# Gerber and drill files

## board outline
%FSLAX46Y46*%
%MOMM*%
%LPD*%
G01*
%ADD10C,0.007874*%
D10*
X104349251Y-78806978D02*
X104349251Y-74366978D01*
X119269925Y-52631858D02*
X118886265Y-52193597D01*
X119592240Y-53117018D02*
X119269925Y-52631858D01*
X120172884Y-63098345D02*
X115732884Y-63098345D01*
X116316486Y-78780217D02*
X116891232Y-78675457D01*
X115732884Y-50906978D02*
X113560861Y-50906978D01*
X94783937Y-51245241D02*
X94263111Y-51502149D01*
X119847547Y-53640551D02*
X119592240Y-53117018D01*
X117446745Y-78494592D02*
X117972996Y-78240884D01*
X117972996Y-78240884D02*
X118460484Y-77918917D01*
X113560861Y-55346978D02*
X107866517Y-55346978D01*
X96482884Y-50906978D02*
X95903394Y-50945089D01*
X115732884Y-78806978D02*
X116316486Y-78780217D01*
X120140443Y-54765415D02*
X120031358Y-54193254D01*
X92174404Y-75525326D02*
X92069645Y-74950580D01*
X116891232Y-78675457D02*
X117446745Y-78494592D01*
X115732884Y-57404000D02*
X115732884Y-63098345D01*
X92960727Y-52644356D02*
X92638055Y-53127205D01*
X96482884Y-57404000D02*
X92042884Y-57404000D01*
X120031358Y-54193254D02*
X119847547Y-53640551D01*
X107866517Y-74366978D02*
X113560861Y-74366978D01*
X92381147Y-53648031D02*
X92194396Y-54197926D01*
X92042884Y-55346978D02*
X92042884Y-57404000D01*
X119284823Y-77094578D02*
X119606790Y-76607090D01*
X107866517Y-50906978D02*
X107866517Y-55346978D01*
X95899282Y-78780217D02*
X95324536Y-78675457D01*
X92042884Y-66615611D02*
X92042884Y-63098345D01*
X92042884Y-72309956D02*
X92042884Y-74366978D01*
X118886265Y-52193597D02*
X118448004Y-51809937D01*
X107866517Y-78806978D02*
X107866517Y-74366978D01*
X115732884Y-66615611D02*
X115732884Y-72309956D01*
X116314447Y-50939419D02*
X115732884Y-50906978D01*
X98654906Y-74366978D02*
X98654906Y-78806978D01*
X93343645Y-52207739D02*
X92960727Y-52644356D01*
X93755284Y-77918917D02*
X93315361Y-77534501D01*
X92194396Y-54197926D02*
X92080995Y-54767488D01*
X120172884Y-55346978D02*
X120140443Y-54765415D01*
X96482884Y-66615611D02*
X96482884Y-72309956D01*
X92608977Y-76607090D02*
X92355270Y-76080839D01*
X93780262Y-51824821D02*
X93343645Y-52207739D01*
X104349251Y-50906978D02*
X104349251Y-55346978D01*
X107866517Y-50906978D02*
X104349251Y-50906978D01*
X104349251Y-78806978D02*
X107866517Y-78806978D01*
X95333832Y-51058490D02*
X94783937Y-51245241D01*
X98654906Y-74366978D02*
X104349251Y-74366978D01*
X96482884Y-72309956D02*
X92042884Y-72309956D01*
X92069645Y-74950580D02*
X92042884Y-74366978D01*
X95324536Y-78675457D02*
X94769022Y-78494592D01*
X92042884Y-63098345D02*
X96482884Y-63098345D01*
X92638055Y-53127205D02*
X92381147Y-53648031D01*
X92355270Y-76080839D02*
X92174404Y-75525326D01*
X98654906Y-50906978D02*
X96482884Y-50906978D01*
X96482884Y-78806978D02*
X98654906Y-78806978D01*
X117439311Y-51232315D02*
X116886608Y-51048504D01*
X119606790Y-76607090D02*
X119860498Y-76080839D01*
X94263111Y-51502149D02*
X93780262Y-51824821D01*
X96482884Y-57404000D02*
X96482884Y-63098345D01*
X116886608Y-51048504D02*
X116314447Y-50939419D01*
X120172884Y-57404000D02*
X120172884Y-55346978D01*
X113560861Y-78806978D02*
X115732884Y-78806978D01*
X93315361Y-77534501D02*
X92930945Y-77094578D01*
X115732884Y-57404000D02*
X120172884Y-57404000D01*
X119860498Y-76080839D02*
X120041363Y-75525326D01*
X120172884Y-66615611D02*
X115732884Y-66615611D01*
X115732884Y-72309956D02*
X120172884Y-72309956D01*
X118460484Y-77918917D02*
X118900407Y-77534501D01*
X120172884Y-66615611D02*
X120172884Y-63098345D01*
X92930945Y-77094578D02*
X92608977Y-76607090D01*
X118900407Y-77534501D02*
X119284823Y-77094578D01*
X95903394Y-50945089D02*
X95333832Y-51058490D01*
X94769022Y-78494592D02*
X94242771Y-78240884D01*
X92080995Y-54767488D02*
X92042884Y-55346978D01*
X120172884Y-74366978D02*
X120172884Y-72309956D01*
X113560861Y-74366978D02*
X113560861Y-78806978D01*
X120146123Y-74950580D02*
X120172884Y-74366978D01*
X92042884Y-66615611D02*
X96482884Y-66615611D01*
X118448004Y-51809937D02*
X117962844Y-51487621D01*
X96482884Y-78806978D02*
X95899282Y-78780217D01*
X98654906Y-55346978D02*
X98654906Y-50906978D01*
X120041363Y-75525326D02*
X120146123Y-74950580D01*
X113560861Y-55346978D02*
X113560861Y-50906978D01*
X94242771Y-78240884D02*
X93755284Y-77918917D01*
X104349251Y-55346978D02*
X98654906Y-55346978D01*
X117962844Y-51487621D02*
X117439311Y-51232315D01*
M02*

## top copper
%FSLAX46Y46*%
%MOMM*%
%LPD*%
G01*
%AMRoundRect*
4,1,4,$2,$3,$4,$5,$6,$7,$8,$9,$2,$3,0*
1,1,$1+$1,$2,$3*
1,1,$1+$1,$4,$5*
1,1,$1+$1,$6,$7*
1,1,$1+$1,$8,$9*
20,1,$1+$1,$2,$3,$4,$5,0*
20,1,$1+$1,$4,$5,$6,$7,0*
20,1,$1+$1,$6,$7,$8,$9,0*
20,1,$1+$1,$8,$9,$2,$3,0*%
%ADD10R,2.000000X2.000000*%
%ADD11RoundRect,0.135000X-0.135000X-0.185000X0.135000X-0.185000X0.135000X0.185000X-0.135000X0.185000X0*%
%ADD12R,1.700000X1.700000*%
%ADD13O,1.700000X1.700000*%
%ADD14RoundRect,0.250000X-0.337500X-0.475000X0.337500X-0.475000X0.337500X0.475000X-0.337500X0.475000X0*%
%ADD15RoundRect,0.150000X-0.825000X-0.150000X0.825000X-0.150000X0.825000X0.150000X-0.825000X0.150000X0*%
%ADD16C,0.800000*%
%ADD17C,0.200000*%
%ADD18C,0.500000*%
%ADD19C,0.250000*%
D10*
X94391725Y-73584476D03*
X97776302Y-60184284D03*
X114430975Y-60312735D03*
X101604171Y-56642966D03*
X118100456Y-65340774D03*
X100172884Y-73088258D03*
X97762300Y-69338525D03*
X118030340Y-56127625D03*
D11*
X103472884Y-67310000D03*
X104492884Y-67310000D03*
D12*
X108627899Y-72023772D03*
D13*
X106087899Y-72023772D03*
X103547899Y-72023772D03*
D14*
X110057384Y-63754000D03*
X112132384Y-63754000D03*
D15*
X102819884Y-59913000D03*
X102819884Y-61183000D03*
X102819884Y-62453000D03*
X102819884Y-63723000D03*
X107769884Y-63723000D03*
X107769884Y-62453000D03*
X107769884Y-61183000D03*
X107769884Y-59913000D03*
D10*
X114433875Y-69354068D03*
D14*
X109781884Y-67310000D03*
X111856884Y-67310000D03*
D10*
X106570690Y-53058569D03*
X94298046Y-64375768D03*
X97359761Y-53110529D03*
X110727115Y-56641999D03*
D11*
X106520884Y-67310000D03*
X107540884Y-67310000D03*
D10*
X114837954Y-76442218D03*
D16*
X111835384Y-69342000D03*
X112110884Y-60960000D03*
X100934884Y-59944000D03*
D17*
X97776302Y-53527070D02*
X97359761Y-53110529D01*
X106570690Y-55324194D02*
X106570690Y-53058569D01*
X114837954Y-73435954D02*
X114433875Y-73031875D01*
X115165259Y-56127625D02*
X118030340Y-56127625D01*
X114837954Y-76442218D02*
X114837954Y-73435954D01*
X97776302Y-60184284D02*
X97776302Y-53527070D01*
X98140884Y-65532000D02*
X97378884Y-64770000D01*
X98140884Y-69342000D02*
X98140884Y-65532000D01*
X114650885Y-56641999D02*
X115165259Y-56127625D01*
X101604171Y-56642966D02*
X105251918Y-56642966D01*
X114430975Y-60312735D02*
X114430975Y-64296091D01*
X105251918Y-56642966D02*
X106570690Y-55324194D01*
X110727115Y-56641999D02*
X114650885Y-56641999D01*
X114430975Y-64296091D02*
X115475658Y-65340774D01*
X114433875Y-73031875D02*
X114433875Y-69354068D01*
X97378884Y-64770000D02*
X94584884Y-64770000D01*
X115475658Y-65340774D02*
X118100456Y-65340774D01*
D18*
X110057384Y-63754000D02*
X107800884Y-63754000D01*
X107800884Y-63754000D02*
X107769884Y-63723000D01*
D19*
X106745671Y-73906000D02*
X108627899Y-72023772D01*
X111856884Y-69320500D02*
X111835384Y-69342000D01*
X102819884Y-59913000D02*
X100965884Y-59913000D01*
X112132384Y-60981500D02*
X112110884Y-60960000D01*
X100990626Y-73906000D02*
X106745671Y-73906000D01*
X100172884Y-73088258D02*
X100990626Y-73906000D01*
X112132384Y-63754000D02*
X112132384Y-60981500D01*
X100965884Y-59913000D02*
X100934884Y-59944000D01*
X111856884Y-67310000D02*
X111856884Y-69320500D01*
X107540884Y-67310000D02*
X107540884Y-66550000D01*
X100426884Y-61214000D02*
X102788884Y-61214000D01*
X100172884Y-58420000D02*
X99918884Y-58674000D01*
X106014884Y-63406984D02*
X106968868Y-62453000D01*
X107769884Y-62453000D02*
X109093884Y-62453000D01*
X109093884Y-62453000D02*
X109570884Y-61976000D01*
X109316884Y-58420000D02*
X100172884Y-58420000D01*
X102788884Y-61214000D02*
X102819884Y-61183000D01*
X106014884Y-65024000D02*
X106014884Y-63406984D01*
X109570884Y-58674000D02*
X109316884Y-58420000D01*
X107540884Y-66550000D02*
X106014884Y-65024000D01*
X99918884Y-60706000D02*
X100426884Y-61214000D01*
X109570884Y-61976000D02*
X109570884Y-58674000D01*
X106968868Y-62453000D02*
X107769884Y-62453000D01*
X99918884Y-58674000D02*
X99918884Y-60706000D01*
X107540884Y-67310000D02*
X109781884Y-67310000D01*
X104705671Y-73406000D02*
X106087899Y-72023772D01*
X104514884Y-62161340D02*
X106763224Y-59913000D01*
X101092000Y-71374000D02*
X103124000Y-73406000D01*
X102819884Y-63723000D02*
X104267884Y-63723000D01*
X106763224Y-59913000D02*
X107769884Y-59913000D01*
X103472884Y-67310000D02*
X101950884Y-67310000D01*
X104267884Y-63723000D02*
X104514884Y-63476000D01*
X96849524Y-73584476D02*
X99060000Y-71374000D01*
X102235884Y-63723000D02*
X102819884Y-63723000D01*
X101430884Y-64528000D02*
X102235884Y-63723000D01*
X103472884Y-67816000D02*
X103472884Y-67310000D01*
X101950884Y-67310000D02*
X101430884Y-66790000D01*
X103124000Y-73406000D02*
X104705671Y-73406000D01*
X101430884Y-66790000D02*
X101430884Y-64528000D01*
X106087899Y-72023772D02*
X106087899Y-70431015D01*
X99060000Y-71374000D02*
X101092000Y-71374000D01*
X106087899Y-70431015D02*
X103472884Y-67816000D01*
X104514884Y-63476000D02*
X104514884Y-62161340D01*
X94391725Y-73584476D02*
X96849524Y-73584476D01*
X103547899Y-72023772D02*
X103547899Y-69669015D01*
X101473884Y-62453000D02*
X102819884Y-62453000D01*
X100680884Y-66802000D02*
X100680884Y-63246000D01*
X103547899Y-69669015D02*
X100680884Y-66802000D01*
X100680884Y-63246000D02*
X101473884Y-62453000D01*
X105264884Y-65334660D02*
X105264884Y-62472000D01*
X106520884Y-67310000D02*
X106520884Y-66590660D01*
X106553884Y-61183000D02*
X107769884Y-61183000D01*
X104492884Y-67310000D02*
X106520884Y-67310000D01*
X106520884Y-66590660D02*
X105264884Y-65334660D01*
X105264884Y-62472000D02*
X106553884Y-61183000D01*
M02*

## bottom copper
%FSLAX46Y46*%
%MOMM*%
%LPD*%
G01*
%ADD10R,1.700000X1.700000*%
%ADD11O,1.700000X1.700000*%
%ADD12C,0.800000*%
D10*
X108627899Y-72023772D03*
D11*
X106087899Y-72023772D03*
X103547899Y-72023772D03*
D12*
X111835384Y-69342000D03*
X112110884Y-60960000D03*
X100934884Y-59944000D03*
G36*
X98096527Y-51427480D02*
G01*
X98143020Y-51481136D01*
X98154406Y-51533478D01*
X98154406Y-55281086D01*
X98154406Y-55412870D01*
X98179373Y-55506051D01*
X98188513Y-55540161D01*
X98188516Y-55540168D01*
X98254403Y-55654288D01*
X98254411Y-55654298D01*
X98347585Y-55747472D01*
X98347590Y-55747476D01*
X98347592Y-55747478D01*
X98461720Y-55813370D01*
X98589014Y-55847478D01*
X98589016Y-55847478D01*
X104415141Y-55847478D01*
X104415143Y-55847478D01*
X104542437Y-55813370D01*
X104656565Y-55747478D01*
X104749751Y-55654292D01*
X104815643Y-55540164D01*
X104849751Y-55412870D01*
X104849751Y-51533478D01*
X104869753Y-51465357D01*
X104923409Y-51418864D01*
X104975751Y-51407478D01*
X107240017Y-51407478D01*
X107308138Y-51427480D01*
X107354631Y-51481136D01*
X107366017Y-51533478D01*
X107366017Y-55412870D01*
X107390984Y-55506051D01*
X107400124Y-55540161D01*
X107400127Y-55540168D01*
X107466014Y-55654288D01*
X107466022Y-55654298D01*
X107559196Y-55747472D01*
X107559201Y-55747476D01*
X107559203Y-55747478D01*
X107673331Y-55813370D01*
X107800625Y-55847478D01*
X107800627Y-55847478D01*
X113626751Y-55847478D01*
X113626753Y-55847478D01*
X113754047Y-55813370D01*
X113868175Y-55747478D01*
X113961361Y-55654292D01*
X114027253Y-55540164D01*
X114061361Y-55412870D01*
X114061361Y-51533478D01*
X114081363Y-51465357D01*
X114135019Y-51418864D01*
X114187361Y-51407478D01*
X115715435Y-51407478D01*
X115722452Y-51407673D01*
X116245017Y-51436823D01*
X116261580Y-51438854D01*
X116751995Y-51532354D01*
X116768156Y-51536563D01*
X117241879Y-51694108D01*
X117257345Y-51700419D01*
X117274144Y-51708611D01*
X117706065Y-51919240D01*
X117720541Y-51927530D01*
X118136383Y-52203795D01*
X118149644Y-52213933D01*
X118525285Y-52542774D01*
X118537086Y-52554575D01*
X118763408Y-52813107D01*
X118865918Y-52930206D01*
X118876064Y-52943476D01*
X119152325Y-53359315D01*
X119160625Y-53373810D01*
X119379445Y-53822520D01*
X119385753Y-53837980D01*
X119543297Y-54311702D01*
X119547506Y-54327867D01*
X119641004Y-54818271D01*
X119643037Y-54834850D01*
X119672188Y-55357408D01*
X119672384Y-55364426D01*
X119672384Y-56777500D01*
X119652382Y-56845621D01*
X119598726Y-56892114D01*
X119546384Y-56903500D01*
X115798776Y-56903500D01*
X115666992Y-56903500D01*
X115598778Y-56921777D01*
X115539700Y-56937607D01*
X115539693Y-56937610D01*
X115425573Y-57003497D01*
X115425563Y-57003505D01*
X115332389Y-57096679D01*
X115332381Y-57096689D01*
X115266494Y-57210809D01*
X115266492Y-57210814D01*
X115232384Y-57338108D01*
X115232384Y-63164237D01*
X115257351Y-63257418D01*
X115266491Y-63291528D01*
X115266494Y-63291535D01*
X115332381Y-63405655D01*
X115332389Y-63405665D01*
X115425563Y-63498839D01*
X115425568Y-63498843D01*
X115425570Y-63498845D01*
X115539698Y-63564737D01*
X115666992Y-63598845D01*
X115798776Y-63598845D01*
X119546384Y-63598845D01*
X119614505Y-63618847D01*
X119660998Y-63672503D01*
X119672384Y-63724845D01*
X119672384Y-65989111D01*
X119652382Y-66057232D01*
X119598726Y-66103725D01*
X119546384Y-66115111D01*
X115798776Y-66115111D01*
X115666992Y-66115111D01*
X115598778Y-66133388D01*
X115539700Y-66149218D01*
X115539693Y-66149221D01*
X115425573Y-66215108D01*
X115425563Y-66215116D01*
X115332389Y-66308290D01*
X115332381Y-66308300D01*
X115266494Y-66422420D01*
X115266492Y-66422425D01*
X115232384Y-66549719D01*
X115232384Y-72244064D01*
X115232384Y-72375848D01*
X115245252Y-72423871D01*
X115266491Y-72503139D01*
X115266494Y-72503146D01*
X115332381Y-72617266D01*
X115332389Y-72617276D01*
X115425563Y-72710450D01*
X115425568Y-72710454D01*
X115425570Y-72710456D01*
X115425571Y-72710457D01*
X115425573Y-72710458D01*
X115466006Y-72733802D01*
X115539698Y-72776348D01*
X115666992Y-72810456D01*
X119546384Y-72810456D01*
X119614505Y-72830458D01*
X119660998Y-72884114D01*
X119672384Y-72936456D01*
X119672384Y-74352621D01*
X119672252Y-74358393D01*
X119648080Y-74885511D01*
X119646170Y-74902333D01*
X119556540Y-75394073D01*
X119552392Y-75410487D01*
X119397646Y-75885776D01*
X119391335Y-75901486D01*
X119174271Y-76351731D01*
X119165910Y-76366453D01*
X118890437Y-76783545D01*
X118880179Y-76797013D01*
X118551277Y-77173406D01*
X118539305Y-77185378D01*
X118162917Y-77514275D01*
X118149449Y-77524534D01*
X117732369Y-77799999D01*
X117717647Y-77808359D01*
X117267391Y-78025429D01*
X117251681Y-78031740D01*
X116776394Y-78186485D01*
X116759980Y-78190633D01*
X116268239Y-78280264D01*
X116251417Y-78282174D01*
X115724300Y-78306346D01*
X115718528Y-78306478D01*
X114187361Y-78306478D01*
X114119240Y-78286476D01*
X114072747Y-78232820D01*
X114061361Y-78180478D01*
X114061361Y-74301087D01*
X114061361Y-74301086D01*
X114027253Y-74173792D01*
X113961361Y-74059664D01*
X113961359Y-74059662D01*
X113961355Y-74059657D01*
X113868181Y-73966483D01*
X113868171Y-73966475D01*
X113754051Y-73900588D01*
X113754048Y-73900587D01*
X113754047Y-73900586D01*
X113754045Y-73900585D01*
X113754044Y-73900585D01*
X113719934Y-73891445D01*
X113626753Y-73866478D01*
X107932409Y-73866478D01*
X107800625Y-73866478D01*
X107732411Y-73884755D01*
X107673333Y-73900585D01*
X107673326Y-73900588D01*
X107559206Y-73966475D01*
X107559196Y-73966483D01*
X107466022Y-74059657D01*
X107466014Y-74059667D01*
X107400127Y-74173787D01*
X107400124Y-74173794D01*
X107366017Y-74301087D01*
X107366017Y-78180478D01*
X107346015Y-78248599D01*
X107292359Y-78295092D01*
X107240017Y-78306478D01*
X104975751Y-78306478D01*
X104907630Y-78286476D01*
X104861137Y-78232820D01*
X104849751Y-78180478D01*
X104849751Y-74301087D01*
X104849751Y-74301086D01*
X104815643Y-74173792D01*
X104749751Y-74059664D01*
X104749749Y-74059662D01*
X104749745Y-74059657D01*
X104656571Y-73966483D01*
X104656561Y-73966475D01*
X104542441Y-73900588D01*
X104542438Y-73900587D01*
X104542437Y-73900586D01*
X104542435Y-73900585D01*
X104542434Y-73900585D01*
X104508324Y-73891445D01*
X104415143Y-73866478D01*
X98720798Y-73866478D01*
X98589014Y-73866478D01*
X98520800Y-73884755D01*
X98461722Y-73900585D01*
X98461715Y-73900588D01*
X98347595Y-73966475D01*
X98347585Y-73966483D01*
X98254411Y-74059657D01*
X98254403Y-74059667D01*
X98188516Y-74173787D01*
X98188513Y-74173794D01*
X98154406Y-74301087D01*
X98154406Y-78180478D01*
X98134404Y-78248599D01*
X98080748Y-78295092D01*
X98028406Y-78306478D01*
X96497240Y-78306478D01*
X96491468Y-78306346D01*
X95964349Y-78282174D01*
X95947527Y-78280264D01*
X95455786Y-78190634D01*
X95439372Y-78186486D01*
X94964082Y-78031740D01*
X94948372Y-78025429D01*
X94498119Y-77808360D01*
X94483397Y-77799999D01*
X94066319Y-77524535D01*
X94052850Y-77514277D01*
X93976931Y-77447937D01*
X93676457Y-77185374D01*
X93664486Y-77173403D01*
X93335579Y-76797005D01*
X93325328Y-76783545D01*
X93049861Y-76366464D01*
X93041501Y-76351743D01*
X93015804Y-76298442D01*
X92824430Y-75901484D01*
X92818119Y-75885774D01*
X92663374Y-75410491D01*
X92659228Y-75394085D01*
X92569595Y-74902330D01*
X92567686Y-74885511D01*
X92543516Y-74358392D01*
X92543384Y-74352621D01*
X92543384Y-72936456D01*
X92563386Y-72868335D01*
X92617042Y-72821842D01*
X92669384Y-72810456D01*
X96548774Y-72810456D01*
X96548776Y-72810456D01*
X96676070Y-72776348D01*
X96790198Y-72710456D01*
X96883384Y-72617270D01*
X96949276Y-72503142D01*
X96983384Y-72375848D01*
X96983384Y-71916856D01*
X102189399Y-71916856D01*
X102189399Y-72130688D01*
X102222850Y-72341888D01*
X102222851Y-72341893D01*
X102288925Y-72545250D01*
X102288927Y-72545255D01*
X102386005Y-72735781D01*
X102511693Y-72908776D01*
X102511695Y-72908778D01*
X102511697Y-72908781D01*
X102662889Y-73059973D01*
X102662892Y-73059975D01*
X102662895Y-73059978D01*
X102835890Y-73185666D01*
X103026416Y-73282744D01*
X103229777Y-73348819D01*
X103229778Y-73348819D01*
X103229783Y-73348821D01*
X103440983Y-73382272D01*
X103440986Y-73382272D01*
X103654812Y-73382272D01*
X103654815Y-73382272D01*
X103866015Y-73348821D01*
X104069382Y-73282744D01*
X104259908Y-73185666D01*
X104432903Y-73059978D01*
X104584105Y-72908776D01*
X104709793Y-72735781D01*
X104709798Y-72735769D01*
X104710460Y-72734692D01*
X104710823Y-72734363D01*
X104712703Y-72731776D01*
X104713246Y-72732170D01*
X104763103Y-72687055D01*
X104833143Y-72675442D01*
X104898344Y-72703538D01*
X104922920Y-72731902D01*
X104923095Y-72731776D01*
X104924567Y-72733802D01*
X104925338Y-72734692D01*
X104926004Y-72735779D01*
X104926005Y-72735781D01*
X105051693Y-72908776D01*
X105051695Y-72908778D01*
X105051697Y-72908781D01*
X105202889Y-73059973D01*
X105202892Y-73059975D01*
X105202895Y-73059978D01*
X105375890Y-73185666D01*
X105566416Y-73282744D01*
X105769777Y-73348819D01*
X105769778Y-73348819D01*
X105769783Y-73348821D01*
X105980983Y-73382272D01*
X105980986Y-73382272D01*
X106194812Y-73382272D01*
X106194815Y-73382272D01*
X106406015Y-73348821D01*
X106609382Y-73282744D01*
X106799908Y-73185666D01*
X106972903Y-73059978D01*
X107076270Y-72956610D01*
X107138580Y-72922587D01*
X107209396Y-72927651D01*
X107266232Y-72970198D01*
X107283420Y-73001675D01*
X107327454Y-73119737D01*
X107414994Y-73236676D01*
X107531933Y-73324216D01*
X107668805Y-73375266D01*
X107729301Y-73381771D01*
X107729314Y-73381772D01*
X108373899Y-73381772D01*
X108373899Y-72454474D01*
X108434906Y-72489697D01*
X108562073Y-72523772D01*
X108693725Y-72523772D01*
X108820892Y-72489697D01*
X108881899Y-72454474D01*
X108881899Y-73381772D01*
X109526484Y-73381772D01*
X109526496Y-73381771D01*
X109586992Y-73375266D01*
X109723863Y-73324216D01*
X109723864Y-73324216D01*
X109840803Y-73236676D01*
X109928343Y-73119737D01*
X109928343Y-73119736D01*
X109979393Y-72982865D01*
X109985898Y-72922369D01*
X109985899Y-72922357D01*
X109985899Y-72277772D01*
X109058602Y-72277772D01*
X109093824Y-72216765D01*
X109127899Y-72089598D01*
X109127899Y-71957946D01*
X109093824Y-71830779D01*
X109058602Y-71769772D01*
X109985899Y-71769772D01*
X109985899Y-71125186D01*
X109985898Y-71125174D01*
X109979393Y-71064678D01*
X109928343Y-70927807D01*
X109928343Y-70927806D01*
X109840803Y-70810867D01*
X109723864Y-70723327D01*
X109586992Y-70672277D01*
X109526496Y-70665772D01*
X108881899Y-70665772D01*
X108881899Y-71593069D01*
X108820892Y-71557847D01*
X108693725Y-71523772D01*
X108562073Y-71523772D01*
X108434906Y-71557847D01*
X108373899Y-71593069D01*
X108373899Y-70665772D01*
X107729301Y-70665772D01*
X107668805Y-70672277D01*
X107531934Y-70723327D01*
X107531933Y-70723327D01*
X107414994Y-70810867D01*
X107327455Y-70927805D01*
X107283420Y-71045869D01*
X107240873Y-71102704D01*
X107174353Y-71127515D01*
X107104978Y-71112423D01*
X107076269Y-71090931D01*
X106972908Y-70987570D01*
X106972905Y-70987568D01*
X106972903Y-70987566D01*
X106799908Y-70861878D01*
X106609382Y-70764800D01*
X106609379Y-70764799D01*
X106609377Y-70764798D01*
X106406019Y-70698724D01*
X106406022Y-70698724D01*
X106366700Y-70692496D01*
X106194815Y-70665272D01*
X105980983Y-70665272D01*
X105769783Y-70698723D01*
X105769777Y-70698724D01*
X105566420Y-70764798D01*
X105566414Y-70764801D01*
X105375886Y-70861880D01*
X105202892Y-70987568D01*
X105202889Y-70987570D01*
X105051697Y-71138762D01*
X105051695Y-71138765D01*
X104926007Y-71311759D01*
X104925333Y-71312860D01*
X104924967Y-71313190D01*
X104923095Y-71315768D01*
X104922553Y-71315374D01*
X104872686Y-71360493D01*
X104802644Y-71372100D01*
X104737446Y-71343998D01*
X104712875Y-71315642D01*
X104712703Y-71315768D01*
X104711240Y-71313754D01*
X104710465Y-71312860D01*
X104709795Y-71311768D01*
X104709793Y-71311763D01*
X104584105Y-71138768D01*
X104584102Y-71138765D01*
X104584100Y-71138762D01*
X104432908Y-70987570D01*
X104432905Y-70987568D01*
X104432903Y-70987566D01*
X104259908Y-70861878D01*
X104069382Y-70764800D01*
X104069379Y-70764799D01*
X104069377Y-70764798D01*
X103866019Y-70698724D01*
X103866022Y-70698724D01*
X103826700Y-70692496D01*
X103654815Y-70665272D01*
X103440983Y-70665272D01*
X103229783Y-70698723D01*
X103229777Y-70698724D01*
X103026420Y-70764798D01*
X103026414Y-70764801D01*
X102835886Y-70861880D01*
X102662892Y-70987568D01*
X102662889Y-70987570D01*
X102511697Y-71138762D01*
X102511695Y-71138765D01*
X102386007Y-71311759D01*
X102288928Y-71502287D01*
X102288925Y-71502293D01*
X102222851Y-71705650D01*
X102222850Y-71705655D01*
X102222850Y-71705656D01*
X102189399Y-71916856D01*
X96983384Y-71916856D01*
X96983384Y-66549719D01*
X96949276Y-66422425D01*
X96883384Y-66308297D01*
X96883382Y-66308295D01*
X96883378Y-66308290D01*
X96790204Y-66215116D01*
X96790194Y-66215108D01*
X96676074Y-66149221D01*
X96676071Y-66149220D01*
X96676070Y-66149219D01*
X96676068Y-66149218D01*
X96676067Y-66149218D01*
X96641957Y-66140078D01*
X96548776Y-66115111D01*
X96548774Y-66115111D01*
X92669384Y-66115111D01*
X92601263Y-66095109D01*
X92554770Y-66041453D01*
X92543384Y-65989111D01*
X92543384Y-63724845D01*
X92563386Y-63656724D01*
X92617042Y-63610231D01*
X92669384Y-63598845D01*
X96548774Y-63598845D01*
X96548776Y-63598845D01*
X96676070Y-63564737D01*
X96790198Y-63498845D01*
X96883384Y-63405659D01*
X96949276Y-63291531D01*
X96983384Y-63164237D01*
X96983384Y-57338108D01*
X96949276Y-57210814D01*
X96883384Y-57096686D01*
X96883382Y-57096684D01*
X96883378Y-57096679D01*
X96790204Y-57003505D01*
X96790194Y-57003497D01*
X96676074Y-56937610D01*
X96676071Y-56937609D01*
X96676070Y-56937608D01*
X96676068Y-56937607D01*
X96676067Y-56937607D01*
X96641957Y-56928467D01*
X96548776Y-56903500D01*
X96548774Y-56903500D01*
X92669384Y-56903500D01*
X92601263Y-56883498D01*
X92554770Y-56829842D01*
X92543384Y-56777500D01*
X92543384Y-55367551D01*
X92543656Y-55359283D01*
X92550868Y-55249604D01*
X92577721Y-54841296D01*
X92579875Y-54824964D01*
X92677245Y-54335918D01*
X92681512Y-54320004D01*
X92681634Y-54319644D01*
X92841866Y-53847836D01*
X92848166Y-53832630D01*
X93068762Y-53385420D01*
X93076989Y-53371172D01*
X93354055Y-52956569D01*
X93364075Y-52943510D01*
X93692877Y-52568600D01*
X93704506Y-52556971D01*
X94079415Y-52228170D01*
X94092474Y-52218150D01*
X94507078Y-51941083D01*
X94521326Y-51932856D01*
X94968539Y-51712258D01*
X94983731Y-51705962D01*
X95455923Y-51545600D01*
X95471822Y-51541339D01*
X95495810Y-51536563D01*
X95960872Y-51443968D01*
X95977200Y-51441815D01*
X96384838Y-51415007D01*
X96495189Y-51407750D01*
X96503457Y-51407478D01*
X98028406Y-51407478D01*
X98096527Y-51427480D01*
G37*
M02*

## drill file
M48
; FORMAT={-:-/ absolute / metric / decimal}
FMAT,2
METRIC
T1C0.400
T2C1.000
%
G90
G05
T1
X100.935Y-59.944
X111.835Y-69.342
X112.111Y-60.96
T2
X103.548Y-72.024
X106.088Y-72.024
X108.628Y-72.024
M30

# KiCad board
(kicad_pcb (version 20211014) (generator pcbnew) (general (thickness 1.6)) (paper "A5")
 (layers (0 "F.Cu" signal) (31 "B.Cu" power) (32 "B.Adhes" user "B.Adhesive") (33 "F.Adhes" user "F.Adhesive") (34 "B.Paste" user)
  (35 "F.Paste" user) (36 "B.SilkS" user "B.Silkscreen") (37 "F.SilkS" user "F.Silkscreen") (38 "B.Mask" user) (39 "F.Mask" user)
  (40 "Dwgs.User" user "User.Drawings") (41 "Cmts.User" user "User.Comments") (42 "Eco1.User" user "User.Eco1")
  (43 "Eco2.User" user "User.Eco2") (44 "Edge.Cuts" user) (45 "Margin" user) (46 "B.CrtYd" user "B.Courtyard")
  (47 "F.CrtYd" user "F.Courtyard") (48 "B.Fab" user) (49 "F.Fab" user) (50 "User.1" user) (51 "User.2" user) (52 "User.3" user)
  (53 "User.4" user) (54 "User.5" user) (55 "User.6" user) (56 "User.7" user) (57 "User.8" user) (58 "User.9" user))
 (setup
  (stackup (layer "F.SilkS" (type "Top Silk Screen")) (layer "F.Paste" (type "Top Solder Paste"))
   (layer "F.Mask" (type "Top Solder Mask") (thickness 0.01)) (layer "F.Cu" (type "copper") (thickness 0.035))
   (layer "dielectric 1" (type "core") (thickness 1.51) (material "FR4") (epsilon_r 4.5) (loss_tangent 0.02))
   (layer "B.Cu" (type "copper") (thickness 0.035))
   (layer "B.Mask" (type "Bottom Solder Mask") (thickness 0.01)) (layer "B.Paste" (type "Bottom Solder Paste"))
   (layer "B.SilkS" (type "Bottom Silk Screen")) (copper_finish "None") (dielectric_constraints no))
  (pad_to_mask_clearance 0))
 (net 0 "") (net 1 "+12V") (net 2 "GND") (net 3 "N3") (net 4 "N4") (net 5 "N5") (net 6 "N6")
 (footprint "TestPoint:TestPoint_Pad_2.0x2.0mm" (layer "F.Cu") (at 94.391725 73.584476)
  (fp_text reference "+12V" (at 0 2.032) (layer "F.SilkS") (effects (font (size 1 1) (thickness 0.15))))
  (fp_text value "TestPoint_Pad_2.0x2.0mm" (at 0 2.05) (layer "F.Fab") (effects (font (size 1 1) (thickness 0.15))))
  (pad "1" smd rect (at 0 0) (size 2 2) (layers "F.Cu" "F.Mask") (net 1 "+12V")))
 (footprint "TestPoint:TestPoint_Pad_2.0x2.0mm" (layer "F.Cu") (at 97.776302 60.184284)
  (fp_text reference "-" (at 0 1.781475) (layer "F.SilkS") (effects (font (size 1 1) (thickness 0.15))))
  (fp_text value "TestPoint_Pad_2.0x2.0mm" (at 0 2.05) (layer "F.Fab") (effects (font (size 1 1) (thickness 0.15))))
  (pad "1" smd rect (at 0 0) (size 2 2) (layers "F.Cu" "F.Mask")))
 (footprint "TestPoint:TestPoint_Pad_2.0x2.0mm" (layer "F.Cu") (at 114.430975 60.312735)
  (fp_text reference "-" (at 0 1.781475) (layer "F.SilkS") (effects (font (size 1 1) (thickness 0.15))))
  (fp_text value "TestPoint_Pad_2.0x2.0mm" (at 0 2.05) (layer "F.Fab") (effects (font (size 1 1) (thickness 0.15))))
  (pad "1" smd rect (at 0 0) (size 2 2) (layers "F.Cu" "F.Mask")))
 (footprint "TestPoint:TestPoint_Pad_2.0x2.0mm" (layer "F.Cu") (at 101.604171 56.642966)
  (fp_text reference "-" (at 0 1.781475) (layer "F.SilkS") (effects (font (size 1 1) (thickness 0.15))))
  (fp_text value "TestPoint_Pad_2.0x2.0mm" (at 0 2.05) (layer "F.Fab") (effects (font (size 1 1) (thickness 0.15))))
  (pad "1" smd rect (at 0 0) (size 2 2) (layers "F.Cu" "F.Mask")))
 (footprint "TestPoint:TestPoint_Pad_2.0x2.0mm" (layer "F.Cu") (at 118.100456 65.340774 -90)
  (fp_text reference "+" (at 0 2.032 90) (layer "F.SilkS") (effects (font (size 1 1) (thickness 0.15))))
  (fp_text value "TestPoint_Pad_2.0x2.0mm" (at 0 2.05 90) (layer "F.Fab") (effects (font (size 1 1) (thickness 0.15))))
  (pad "1" smd rect (at 0 0 270) (size 2 2) (layers "F.Cu" "F.Mask")))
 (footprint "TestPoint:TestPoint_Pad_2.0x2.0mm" (layer "F.Cu") (at 100.172884 73.088258 180)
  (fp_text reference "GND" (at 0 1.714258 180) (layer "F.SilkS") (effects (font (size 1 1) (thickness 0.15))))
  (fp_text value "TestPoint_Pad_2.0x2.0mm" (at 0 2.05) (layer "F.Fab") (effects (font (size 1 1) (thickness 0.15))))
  (pad "1" smd rect (at 0 0 180) (size 2 2) (layers "F.Cu" "F.Mask") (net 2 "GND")))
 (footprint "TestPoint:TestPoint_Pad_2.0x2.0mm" (layer "F.Cu") (at 97.7623 69.338525)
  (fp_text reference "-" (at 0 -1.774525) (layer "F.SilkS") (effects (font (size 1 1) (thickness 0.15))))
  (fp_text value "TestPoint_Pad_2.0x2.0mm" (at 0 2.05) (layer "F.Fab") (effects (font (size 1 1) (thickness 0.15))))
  (pad "1" smd rect (at 0 0) (size 2 2) (layers "F.Cu" "F.Mask")))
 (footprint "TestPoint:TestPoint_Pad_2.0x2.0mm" (layer "F.Cu") (at 118.03034 56.127625 -90)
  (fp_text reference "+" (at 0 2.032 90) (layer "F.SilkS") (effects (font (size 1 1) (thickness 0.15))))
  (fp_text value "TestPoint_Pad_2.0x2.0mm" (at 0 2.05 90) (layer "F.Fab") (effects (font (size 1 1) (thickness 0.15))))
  (pad "1" smd rect (at 0 0 270) (size 2 2) (layers "F.Cu" "F.Mask")))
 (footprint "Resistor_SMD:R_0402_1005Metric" (layer "F.Cu") (at 103.982884 67.31)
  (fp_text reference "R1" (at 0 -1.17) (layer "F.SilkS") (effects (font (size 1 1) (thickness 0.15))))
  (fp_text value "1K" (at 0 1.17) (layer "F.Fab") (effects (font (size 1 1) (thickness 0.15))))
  (pad "1" smd roundrect (at -0.51 0) (size 0.54 0.64) (layers "F.Cu" "F.Paste" "F.Mask") (roundrect_rratio 0.25) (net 1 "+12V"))
  (pad "2" smd roundrect (at 0.51 0) (size 0.54 0.64) (layers "F.Cu" "F.Paste" "F.Mask") (roundrect_rratio 0.25) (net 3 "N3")))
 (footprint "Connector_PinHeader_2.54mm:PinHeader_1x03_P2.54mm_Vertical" (layer "F.Cu") (at 108.627899 72.023772 -90)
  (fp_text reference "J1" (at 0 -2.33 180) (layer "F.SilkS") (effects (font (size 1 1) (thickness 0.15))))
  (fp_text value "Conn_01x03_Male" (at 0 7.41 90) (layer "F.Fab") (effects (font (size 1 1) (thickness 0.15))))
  (pad "1" thru_hole rect (at 0 0 270) (size 1.7 1.7) (drill 1) (layers *.Cu *.Mask) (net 2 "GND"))
  (pad "2" thru_hole oval (at 0 2.54 270) (size 1.7 1.7) (drill 1) (layers *.Cu *.Mask) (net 1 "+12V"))
  (pad "3" thru_hole oval (at 0 5.08 270) (size 1.7 1.7) (drill 1) (layers *.Cu *.Mask) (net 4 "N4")))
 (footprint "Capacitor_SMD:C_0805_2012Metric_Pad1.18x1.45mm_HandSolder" (layer "F.Cu") (at 111.094884 63.754)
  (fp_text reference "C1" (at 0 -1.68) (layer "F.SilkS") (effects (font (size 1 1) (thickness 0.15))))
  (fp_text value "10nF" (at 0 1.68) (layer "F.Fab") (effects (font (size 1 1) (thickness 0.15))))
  (pad "1" smd roundrect (at -1.0375 0) (size 1.175 1.45) (layers "F.Cu" "F.Paste" "F.Mask") (roundrect_rratio 0.2127659574) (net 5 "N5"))
  (pad "2" smd roundrect (at 1.0375 0) (size 1.175 1.45) (layers "F.Cu" "F.Paste" "F.Mask") (roundrect_rratio 0.2127659574) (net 2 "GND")))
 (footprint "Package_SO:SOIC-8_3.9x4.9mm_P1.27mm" (layer "F.Cu") (at 105.294884 61.818)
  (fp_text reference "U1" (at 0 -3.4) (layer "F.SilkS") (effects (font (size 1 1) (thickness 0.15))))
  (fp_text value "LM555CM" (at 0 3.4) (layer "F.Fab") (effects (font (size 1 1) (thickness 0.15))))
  (pad "1" smd roundrect (at -2.475 -1.905) (size 1.95 0.6) (layers "F.Cu" "F.Paste" "F.Mask") (roundrect_rratio 0.25) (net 2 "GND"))
  (pad "2" smd roundrect (at -2.475 -0.635) (size 1.95 0.6) (layers "F.Cu" "F.Paste" "F.Mask") (roundrect_rratio 0.25) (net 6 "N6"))
  (pad "3" smd roundrect (at -2.475 0.635) (size 1.95 0.6) (layers "F.Cu" "F.Paste" "F.Mask") (roundrect_rratio 0.25) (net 4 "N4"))
  (pad "4" smd roundrect (at -2.475 1.905) (size 1.95 0.6) (layers "F.Cu" "F.Paste" "F.Mask") (roundrect_rratio 0.25) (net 1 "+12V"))
  (pad "5" smd roundrect (at 2.475 1.905) (size 1.95 0.6) (layers "F.Cu" "F.Paste" "F.Mask") (roundrect_rratio 0.25) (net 5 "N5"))
  (pad "6" smd roundrect (at 2.475 0.635) (size 1.95 0.6) (layers "F.Cu" "F.Paste" "F.Mask") (roundrect_rratio 0.25) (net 6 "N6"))
  (pad "7" smd roundrect (at 2.475 -0.635) (size 1.95 0.6) (layers "F.Cu" "F.Paste" "F.Mask") (roundrect_rratio 0.25) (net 3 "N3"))
  (pad "8" smd roundrect (at 2.475 -1.905) (size 1.95 0.6) (layers "F.Cu" "F.Paste" "F.Mask") (roundrect_rratio 0.25) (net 1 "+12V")))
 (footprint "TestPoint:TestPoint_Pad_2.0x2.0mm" (layer "F.Cu") (at 114.433875 69.354068)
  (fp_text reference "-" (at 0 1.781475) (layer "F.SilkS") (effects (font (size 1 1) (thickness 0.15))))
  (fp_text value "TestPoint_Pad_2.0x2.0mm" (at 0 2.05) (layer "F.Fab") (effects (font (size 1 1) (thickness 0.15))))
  (pad "1" smd rect (at 0 0) (size 2 2) (layers "F.Cu" "F.Mask")))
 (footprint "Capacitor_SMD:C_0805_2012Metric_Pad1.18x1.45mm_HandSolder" (layer "F.Cu") (at 110.819384 67.31)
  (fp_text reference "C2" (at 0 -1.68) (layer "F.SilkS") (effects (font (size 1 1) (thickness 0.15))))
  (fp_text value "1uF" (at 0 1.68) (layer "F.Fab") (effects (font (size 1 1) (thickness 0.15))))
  (pad "1" smd roundrect (at -1.0375 0) (size 1.175 1.45) (layers "F.Cu" "F.Paste" "F.Mask") (roundrect_rratio 0.2127659574) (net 6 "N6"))
  (pad "2" smd roundrect (at 1.0375 0) (size 1.175 1.45) (layers "F.Cu" "F.Paste" "F.Mask") (roundrect_rratio 0.2127659574) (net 2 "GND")))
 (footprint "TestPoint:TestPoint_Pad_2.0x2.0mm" (layer "F.Cu") (at 106.57069 53.058569)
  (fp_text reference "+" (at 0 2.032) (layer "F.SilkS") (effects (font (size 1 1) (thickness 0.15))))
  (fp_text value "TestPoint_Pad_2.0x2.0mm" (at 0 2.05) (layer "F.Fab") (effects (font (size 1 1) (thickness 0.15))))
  (pad "1" smd rect (at 0 0) (size 2 2) (layers "F.Cu" "F.Mask")))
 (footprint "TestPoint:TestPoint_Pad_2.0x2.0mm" (layer "F.Cu") (at 94.298046 64.375768)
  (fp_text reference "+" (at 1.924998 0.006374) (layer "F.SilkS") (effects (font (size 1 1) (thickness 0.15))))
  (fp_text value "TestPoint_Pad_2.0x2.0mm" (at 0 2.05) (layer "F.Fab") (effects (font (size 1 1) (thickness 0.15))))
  (pad "1" smd rect (at 0 0) (size 2 2) (layers "F.Cu" "F.Mask")))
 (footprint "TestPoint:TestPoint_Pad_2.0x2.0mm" (layer "F.Cu") (at 97.359761 53.110529)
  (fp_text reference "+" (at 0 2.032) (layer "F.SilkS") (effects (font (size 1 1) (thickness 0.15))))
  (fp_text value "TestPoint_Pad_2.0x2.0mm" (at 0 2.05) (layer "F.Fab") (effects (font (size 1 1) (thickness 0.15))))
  (pad "1" smd rect (at 0 0) (size 2 2) (layers "F.Cu" "F.Mask")))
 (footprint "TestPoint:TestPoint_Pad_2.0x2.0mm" (layer "F.Cu") (at 110.727115 56.641999)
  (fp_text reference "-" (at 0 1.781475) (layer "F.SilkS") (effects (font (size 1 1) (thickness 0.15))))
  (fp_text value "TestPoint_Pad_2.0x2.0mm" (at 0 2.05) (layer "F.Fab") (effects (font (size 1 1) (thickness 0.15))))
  (pad "1" smd rect (at 0 0) (size 2 2) (layers "F.Cu" "F.Mask")))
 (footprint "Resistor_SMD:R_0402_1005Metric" (layer "F.Cu") (at 107.030884 67.31)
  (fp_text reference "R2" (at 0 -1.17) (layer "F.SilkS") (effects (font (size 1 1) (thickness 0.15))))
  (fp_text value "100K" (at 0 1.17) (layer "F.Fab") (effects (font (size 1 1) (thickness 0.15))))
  (pad "1" smd roundrect (at -0.51 0) (size 0.54 0.64) (layers "F.Cu" "F.Paste" "F.Mask") (roundrect_rratio 0.25) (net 3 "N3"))
  (pad "2" smd roundrect (at 0.51 0) (size 0.54 0.64) (layers "F.Cu" "F.Paste" "F.Mask") (roundrect_rratio 0.25) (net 6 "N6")))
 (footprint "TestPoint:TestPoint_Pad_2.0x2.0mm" (layer "F.Cu") (at 114.837954 76.442218 90)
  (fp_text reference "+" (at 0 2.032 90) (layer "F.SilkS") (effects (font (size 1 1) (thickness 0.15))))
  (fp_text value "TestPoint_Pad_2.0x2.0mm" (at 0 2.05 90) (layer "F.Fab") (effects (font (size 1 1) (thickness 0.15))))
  (pad "1" smd rect (at 0 0 90) (size 2 2) (layers "F.Cu" "F.Mask")))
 (gr_line (start 104.349251 78.806978) (end 104.349251 74.366978) (layer "Edge.Cuts") (width 0.007874))
 (gr_line (start 119.269925 52.631858) (end 118.886265 52.193597) (layer "Edge.Cuts") (width 0.007874))
 (gr_line (start 119.59224 53.117018) (end 119.269925 52.631858) (layer "Edge.Cuts") (width 0.007874))
 (gr_line (start 120.172884 63.098345) (end 115.732884 63.098345) (layer "Edge.Cuts") (width 0.007874))
 (gr_line (start 116.316486 78.780217) (end 116.891232 78.675457) (layer "Edge.Cuts") (width 0.007874))
 (gr_line (start 115.732884 50.906978) (end 113.560861 50.906978) (layer "Edge.Cuts") (width 0.007874))
 (gr_line (start 94.783937 51.245241) (end 94.263111 51.502149) (layer "Edge.Cuts") (width 0.007874))
 (gr_line (start 119.847547 53.640551) (end 119.59224 53.117018) (layer "Edge.Cuts") (width 0.007874))
 (gr_line (start 117.446745 78.494592) (end 117.972996 78.240884) (layer "Edge.Cuts") (width 0.007874))
 (gr_line (start 117.972996 78.240884) (end 118.460484 77.918917) (layer "Edge.Cuts") (width 0.007874))
 (gr_line (start 113.560861 55.346978) (end 107.866517 55.346978) (layer "Edge.Cuts") (width 0.007874))
 (gr_line (start 96.482884 50.906978) (end 95.903394 50.945089) (layer "Edge.Cuts") (width 0.007874))
 (gr_line (start 115.732884 78.806978) (end 116.316486 78.780217) (layer "Edge.Cuts") (width 0.007874))
 (gr_line (start 120.140443 54.765415) (end 120.031358 54.193254) (layer "Edge.Cuts") (width 0.007874))
 (gr_line (start 92.174404 75.525326) (end 92.069645 74.95058) (layer "Edge.Cuts") (width 0.007874))
 (gr_line (start 116.891232 78.675457) (end 117.446745 78.494592) (layer "Edge.Cuts") (width 0.007874))
 (gr_line (start 115.732884 57.404) (end 115.732884 63.098345) (layer "Edge.Cuts") (width 0.007874))
 (gr_line (start 92.960727 52.644356) (end 92.638055 53.127205) (layer "Edge.Cuts") (width 0.007874))
 (gr_line (start 96.482884 57.404) (end 92.042884 57.404) (layer "Edge.Cuts") (width 0.007874))
 (gr_line (start 120.031358 54.193254) (end 119.847547 53.640551) (layer "Edge.Cuts") (width 0.007874))
 (gr_line (start 107.866517 74.366978) (end 113.560861 74.366978) (layer "Edge.Cuts") (width 0.007874))
 (gr_line (start 92.381147 53.648031) (end 92.194396 54.197926) (layer "Edge.Cuts") (width 0.007874))
 (gr_line (start 92.042884 55.346978) (end 92.042884 57.404) (layer "Edge.Cuts") (width 0.007874))
 (gr_line (start 119.284823 77.094578) (end 119.60679 76.60709) (layer "Edge.Cuts") (width 0.007874))
 (gr_line (start 107.866517 50.906978) (end 107.866517 55.346978) (layer "Edge.Cuts") (width 0.007874))
 (gr_line (start 95.899282 78.780217) (end 95.324536 78.675457) (layer "Edge.Cuts") (width 0.007874))
 (gr_line (start 92.042884 66.615611) (end 92.042884 63.098345) (layer "Edge.Cuts") (width 0.007874))
 (gr_line (start 92.042884 72.309956) (end 92.042884 74.366978) (layer "Edge.Cuts") (width 0.007874))
 (gr_line (start 118.886265 52.193597) (end 118.448004 51.809937) (layer "Edge.Cuts") (width 0.007874))
 (gr_line (start 107.866517 78.806978) (end 107.866517 74.366978) (layer "Edge.Cuts") (width 0.007874))
 (gr_line (start 115.732884 66.615611) (end 115.732884 72.309956) (layer "Edge.Cuts") (width 0.007874))
 (gr_line (start 116.314447 50.939419) (end 115.732884 50.906978) (layer "Edge.Cuts") (width 0.007874))
 (gr_line (start 98.654906 74.366978) (end 98.654906 78.806978) (layer "Edge.Cuts") (width 0.007874))
 (gr_line (start 93.343645 52.207739) (end 92.960727 52.644356) (layer "Edge.Cuts") (width 0.007874))
 (gr_line (start 93.755284 77.918917) (end 93.315361 77.534501) (layer "Edge.Cuts") (width 0.007874))
 (gr_line (start 92.194396 54.197926) (end 92.080995 54.767488) (layer "Edge.Cuts") (width 0.007874))
 (gr_line (start 120.172884 55.346978) (end 120.140443 54.765415) (layer "Edge.Cuts") (width 0.007874))
 (gr_line (start 96.482884 66.615611) (end 96.482884 72.309956) (layer "Edge.Cuts") (width 0.007874))
 (gr_line (start 92.608977 76.60709) (end 92.35527 76.080839) (layer "Edge.Cuts") (width 0.007874))
 (gr_line (start 93.780262 51.824821) (end 93.343645 52.207739) (layer "Edge.Cuts") (width 0.007874))
 (gr_line (start 104.349251 50.906978) (end 104.349251 55.346978) (layer "Edge.Cuts") (width 0.007874))
 (gr_line (start 107.866517 50.906978) (end 104.349251 50.906978) (layer "Edge.Cuts") (width 0.007874))
 (gr_line (start 104.349251 78.806978) (end 107.866517 78.806978) (layer "Edge.Cuts") (width 0.007874))
 (gr_line (start 95.333832 51.05849) (end 94.783937 51.245241) (layer "Edge.Cuts") (width 0.007874))
 (gr_line (start 98.654906 74.366978) (end 104.349251 74.366978) (layer "Edge.Cuts") (width 0.007874))
 (gr_line (start 96.482884 72.309956) (end 92.042884 72.309956) (layer "Edge.Cuts") (width 0.007874))
 (gr_line (start 92.069645 74.95058) (end 92.042884 74.366978) (layer "Edge.Cuts") (width 0.007874))
 (gr_line (start 95.324536 78.675457) (end 94.769022 78.494592) (layer "Edge.Cuts") (width 0.007874))
 (gr_line (start 92.042884 63.098345) (end 96.482884 63.098345) (layer "Edge.Cuts") (width 0.007874))
 (gr_line (start 92.638055 53.127205) (end 92.381147 53.648031) (layer "Edge.Cuts") (width 0.007874))
 (gr_line (start 92.35527 76.080839) (end 92.174404 75.525326) (layer "Edge.Cuts") (width 0.007874))
 (gr_line (start 98.654906 50.906978) (end 96.482884 50.906978) (layer "Edge.Cuts") (width 0.007874))
 (gr_line (start 96.482884 78.806978) (end 98.654906 78.806978) (layer "Edge.Cuts") (width 0.007874))
 (gr_line (start 117.439311 51.232315) (end 116.886608 51.048504) (layer "Edge.Cuts") (width 0.007874))
 (gr_line (start 119.60679 76.60709) (end 119.860498 76.080839) (layer "Edge.Cuts") (width 0.007874))
 (gr_line (start 94.263111 51.502149) (end 93.780262 51.824821) (layer "Edge.Cuts") (width 0.007874))
 (gr_line (start 96.482884 57.404) (end 96.482884 63.098345) (layer "Edge.Cuts") (width 0.007874))
 (gr_line (start 116.886608 51.048504) (end 116.314447 50.939419) (layer "Edge.Cuts") (width 0.007874))
 (gr_line (start 120.172884 57.404) (end 120.172884 55.346978) (layer "Edge.Cuts") (width 0.007874))
 (gr_line (start 113.560861 78.806978) (end 115.732884 78.806978) (layer "Edge.Cuts") (width 0.007874))
 (gr_line (start 93.315361 77.534501) (end 92.930945 77.094578) (layer "Edge.Cuts") (width 0.007874))
 (gr_line (start 115.732884 57.404) (end 120.172884 57.404) (layer "Edge.Cuts") (width 0.007874))
 (gr_line (start 119.860498 76.080839) (end 120.041363 75.525326) (layer "Edge.Cuts") (width 0.007874))
 (gr_line (start 120.172884 66.615611) (end 115.732884 66.615611) (layer "Edge.Cuts") (width 0.007874))
 (gr_line (start 115.732884 72.309956) (end 120.172884 72.309956) (layer "Edge.Cuts") (width 0.007874))
 (gr_line (start 118.460484 77.918917) (end 118.900407 77.534501) (layer "Edge.Cuts") (width 0.007874))
 (gr_line (start 120.172884 66.615611) (end 120.172884 63.098345) (layer "Edge.Cuts") (width 0.007874))
 (gr_line (start 92.930945 77.094578) (end 92.608977 76.60709) (layer "Edge.Cuts") (width 0.007874))
 (gr_line (start 118.900407 77.534501) (end 119.284823 77.094578) (layer "Edge.Cuts") (width 0.007874))
 (gr_line (start 95.903394 50.945089) (end 95.333832 51.05849) (layer "Edge.Cuts") (width 0.007874))
 (gr_line (start 94.769022 78.494592) (end 94.242771 78.240884) (layer "Edge.Cuts") (width 0.007874))
 (gr_line (start 92.080995 54.767488) (end 92.042884 55.346978) (layer "Edge.Cuts") (width 0.007874))
 (gr_line (start 120.172884 74.366978) (end 120.172884 72.309956) (layer "Edge.Cuts") (width 0.007874))
 (gr_line (start 113.560861 74.366978) (end 113.560861 78.806978) (layer "Edge.Cuts") (width 0.007874))
 (gr_line (start 120.146123 74.95058) (end 120.172884 74.366978) (layer "Edge.Cuts") (width 0.007874))
 (gr_line (start 92.042884 66.615611) (end 96.482884 66.615611) (layer "Edge.Cuts") (width 0.007874))
 (gr_line (start 118.448004 51.809937) (end 117.962844 51.487621) (layer "Edge.Cuts") (width 0.007874))
 (gr_line (start 96.482884 78.806978) (end 95.899282 78.780217) (layer "Edge.Cuts") (width 0.007874))
 (gr_line (start 98.654906 55.346978) (end 98.654906 50.906978) (layer "Edge.Cuts") (width 0.007874))
 (gr_line (start 120.041363 75.525326) (end 120.146123 74.95058) (layer "Edge.Cuts") (width 0.007874))
 (gr_line (start 113.560861 55.346978) (end 113.560861 50.906978) (layer "Edge.Cuts") (width 0.007874))
 (gr_line (start 94.242771 78.240884) (end 93.755284 77.918917) (layer "Edge.Cuts") (width 0.007874))
 (gr_line (start 104.349251 55.346978) (end 98.654906 55.346978) (layer "Edge.Cuts") (width 0.007874))
 (gr_line (start 117.962844 51.487621) (end 117.439311 51.232315) (layer "Edge.Cuts") (width 0.007874))
 (segment (start 97.776302 53.52707) (end 97.359761 53.110529) (width 0.2) (layer "F.Cu") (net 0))
 (segment (start 106.57069 55.324194) (end 106.57069 53.058569) (width 0.2) (layer "F.Cu") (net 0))
 (segment (start 114.837954 73.435954) (end 114.433875 73.031875) (width 0.2) (layer "F.Cu") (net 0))
 (segment (start 115.165259 56.127625) (end 118.03034 56.127625) (width 0.2) (layer "F.Cu") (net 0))
 (segment (start 114.837954 76.442218) (end 114.837954 73.435954) (width 0.2) (layer "F.Cu") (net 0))
 (segment (start 97.776302 60.184284) (end 97.776302 53.52707) (width 0.2) (layer "F.Cu") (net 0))
 (segment (start 98.140884 65.532) (end 97.378884 64.77) (width 0.2) (layer "F.Cu") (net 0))
 (segment (start 98.140884 69.342) (end 98.140884 65.532) (width 0.2) (layer "F.Cu") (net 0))
 (segment (start 114.650885 56.641999) (end 115.165259 56.127625) (width 0.2) (layer "F.Cu") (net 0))
 (segment (start 101.604171 56.642966) (end 105.251918 56.642966) (width 0.2) (layer "F.Cu") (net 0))
 (segment (start 114.430975 60.312735) (end 114.430975 64.296091) (width 0.2) (layer "F.Cu") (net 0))
 (segment (start 105.251918 56.642966) (end 106.57069 55.324194) (width 0.2) (layer "F.Cu") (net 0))
 (segment (start 110.727115 56.641999) (end 114.650885 56.641999) (width 0.2) (layer "F.Cu") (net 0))
 (segment (start 114.430975 64.296091) (end 115.475658 65.340774) (width 0.2) (layer "F.Cu") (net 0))
 (segment (start 114.433875 73.031875) (end 114.433875 69.354068) (width 0.2) (layer "F.Cu") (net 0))
 (segment (start 97.378884 64.77) (end 94.584884 64.77) (width 0.2) (layer "F.Cu") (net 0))
 (segment (start 115.475658 65.340774) (end 118.100456 65.340774) (width 0.2) (layer "F.Cu") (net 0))
 (segment (start 110.057384 63.754) (end 107.800884 63.754) (width 0.5) (layer "F.Cu") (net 5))
 (segment (start 107.800884 63.754) (end 107.769884 63.723) (width 0.5) (layer "F.Cu") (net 5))
 (segment (start 106.745671 73.906) (end 108.627899 72.023772) (width 0.25) (layer "F.Cu") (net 2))
 (segment (start 111.856884 69.3205) (end 111.835384 69.342) (width 0.25) (layer "F.Cu") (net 2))
 (segment (start 102.819884 59.913) (end 100.965884 59.913) (width 0.25) (layer "F.Cu") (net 2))
 (segment (start 112.132384 60.9815) (end 112.110884 60.96) (width 0.25) (layer "F.Cu") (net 2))
 (segment (start 100.990626 73.906) (end 106.745671 73.906) (width 0.25) (layer "F.Cu") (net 2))
 (segment (start 100.172884 73.088258) (end 100.990626 73.906) (width 0.25) (layer "F.Cu") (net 2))
 (segment (start 112.132384 63.754) (end 112.132384 60.9815) (width 0.25) (layer "F.Cu") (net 2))
 (segment (start 100.965884 59.913) (end 100.934884 59.944) (width 0.25) (layer "F.Cu") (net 2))
 (segment (start 111.856884 67.31) (end 111.856884 69.3205) (width 0.25) (layer "F.Cu") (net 2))
 (via (at 111.835384 69.342) (size 0.8) (drill 0.4) (layers "F.Cu" "B.Cu") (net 2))
 (via (at 112.110884 60.96) (size 0.8) (drill 0.4) (layers "F.Cu" "B.Cu") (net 2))
 (via (at 100.934884 59.944) (size 0.8) (drill 0.4) (layers "F.Cu" "B.Cu") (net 2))
 (segment (start 107.540884 67.31) (end 107.540884 66.55) (width 0.25) (layer "F.Cu") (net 6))
 (segment (start 100.426884 61.214) (end 102.788884 61.214) (width 0.25) (layer "F.Cu") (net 6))
 (segment (start 100.172884 58.42) (end 99.918884 58.674) (width 0.25) (layer "F.Cu") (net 6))
 (segment (start 106.014884 63.406984) (end 106.968868 62.453) (width 0.25) (layer "F.Cu") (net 6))
 (segment (start 107.769884 62.453) (end 109.093884 62.453) (width 0.25) (layer "F.Cu") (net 6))
 (segment (start 109.093884 62.453) (end 109.570884 61.976) (width 0.25) (layer "F.Cu") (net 6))
 (segment (start 109.316884 58.42) (end 100.172884 58.42) (width 0.25) (layer "F.Cu") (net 6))
 (segment (start 102.788884 61.214) (end 102.819884 61.183) (width 0.25) (layer "F.Cu") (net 6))
 (segment (start 106.014884 65.024) (end 106.014884 63.406984) (width 0.25) (layer "F.Cu") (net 6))
 (segment (start 109.570884 58.674) (end 109.316884 58.42) (width 0.25) (layer "F.Cu") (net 6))
 (segment (start 107.540884 66.55) (end 106.014884 65.024) (width 0.25) (layer "F.Cu") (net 6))
 (segment (start 99.918884 60.706) (end 100.426884 61.214) (width 0.25) (layer "F.Cu") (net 6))
 (segment (start 109.570884 61.976) (end 109.570884 58.674) (width 0.25) (layer "F.Cu") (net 6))
 (segment (start 106.968868 62.453) (end 107.769884 62.453) (width 0.25) (layer "F.Cu") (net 6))
 (segment (start 99.918884 58.674) (end 99.918884 60.706) (width 0.25) (layer "F.Cu") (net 6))
 (segment (start 107.540884 67.31) (end 109.781884 67.31) (width 0.25) (layer "F.Cu") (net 6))
 (segment (start 104.705671 73.406) (end 106.087899 72.023772) (width 0.25) (layer "F.Cu") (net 1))
 (segment (start 104.514884 62.16134) (end 106.763224 59.913) (width 0.25) (layer "F.Cu") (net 1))
 (segment (start 101.092 71.374) (end 103.124 73.406) (width 0.25) (layer "F.Cu") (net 1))
 (segment (start 102.819884 63.723) (end 104.267884 63.723) (width 0.25) (layer "F.Cu") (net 1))
 (segment (start 106.763224 59.913) (end 107.769884 59.913) (width 0.25) (layer "F.Cu") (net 1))
 (segment (start 103.472884 67.31) (end 101.950884 67.31) (width 0.25) (layer "F.Cu") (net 1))
 (segment (start 104.267884 63.723) (end 104.514884 63.476) (width 0.25) (layer "F.Cu") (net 1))
 (segment (start 96.849524 73.584476) (end 99.06 71.374) (width 0.25) (layer "F.Cu") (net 1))
 (segment (start 102.235884 63.723) (end 102.819884 63.723) (width 0.25) (layer "F.Cu") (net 1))
 (segment (start 101.430884 64.528) (end 102.235884 63.723) (width 0.25) (layer "F.Cu") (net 1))
 (segment (start 103.472884 67.816) (end 103.472884 67.31) (width 0.25) (layer "F.Cu") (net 1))
 (segment (start 101.950884 67.31) (end 101.430884 66.79) (width 0.25) (layer "F.Cu") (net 1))
 (segment (start 103.124 73.406) (end 104.705671 73.406) (width 0.25) (layer "F.Cu") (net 1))
 (segment (start 101.430884 66.79) (end 101.430884 64.528) (width 0.25) (layer "F.Cu") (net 1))
 (segment (start 106.087899 72.023772) (end 106.087899 70.431015) (width 0.25) (layer "F.Cu") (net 1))
 (segment (start 99.06 71.374) (end 101.092 71.374) (width 0.25) (layer "F.Cu") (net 1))
 (segment (start 106.087899 70.431015) (end 103.472884 67.816) (width 0.25) (layer "F.Cu") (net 1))
 (segment (start 104.514884 63.476) (end 104.514884 62.16134) (width 0.25) (layer "F.Cu") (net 1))
 (segment (start 94.391725 73.584476) (end 96.849524 73.584476) (width 0.25) (layer "F.Cu") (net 1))
 (segment (start 103.547899 72.023772) (end 103.547899 69.669015) (width 0.25) (layer "F.Cu") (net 4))
 (segment (start 101.473884 62.453) (end 102.819884 62.453) (width 0.25) (layer "F.Cu") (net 4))
 (segment (start 100.680884 66.802) (end 100.680884 63.246) (width 0.25) (layer "F.Cu") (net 4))
 (segment (start 103.547899 69.669015) (end 100.680884 66.802) (width 0.25) (layer "F.Cu") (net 4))
 (segment (start 100.680884 63.246) (end 101.473884 62.453) (width 0.25) (layer "F.Cu") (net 4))
 (segment (start 105.264884 65.33466) (end 105.264884 62.472) (width 0.25) (layer "F.Cu") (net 3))
 (segment (start 106.520884 67.31) (end 106.520884 66.59066) (width 0.25) (layer "F.Cu") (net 3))
 (segment (start 106.553884 61.183) (end 107.769884 61.183) (width 0.25) (layer "F.Cu") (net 3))
 (segment (start 104.492884 67.31) (end 106.520884 67.31) (width 0.25) (layer "F.Cu") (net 3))
 (segment (start 106.520884 66.59066) (end 105.264884 65.33466) (width 0.25) (layer "F.Cu") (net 3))
 (segment (start 105.264884 62.472) (end 106.553884 61.183) (width 0.25) (layer "F.Cu") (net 3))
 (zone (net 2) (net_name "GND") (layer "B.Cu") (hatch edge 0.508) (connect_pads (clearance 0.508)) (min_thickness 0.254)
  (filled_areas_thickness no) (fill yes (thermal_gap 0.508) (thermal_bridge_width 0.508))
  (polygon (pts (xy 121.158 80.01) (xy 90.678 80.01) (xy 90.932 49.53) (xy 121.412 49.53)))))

